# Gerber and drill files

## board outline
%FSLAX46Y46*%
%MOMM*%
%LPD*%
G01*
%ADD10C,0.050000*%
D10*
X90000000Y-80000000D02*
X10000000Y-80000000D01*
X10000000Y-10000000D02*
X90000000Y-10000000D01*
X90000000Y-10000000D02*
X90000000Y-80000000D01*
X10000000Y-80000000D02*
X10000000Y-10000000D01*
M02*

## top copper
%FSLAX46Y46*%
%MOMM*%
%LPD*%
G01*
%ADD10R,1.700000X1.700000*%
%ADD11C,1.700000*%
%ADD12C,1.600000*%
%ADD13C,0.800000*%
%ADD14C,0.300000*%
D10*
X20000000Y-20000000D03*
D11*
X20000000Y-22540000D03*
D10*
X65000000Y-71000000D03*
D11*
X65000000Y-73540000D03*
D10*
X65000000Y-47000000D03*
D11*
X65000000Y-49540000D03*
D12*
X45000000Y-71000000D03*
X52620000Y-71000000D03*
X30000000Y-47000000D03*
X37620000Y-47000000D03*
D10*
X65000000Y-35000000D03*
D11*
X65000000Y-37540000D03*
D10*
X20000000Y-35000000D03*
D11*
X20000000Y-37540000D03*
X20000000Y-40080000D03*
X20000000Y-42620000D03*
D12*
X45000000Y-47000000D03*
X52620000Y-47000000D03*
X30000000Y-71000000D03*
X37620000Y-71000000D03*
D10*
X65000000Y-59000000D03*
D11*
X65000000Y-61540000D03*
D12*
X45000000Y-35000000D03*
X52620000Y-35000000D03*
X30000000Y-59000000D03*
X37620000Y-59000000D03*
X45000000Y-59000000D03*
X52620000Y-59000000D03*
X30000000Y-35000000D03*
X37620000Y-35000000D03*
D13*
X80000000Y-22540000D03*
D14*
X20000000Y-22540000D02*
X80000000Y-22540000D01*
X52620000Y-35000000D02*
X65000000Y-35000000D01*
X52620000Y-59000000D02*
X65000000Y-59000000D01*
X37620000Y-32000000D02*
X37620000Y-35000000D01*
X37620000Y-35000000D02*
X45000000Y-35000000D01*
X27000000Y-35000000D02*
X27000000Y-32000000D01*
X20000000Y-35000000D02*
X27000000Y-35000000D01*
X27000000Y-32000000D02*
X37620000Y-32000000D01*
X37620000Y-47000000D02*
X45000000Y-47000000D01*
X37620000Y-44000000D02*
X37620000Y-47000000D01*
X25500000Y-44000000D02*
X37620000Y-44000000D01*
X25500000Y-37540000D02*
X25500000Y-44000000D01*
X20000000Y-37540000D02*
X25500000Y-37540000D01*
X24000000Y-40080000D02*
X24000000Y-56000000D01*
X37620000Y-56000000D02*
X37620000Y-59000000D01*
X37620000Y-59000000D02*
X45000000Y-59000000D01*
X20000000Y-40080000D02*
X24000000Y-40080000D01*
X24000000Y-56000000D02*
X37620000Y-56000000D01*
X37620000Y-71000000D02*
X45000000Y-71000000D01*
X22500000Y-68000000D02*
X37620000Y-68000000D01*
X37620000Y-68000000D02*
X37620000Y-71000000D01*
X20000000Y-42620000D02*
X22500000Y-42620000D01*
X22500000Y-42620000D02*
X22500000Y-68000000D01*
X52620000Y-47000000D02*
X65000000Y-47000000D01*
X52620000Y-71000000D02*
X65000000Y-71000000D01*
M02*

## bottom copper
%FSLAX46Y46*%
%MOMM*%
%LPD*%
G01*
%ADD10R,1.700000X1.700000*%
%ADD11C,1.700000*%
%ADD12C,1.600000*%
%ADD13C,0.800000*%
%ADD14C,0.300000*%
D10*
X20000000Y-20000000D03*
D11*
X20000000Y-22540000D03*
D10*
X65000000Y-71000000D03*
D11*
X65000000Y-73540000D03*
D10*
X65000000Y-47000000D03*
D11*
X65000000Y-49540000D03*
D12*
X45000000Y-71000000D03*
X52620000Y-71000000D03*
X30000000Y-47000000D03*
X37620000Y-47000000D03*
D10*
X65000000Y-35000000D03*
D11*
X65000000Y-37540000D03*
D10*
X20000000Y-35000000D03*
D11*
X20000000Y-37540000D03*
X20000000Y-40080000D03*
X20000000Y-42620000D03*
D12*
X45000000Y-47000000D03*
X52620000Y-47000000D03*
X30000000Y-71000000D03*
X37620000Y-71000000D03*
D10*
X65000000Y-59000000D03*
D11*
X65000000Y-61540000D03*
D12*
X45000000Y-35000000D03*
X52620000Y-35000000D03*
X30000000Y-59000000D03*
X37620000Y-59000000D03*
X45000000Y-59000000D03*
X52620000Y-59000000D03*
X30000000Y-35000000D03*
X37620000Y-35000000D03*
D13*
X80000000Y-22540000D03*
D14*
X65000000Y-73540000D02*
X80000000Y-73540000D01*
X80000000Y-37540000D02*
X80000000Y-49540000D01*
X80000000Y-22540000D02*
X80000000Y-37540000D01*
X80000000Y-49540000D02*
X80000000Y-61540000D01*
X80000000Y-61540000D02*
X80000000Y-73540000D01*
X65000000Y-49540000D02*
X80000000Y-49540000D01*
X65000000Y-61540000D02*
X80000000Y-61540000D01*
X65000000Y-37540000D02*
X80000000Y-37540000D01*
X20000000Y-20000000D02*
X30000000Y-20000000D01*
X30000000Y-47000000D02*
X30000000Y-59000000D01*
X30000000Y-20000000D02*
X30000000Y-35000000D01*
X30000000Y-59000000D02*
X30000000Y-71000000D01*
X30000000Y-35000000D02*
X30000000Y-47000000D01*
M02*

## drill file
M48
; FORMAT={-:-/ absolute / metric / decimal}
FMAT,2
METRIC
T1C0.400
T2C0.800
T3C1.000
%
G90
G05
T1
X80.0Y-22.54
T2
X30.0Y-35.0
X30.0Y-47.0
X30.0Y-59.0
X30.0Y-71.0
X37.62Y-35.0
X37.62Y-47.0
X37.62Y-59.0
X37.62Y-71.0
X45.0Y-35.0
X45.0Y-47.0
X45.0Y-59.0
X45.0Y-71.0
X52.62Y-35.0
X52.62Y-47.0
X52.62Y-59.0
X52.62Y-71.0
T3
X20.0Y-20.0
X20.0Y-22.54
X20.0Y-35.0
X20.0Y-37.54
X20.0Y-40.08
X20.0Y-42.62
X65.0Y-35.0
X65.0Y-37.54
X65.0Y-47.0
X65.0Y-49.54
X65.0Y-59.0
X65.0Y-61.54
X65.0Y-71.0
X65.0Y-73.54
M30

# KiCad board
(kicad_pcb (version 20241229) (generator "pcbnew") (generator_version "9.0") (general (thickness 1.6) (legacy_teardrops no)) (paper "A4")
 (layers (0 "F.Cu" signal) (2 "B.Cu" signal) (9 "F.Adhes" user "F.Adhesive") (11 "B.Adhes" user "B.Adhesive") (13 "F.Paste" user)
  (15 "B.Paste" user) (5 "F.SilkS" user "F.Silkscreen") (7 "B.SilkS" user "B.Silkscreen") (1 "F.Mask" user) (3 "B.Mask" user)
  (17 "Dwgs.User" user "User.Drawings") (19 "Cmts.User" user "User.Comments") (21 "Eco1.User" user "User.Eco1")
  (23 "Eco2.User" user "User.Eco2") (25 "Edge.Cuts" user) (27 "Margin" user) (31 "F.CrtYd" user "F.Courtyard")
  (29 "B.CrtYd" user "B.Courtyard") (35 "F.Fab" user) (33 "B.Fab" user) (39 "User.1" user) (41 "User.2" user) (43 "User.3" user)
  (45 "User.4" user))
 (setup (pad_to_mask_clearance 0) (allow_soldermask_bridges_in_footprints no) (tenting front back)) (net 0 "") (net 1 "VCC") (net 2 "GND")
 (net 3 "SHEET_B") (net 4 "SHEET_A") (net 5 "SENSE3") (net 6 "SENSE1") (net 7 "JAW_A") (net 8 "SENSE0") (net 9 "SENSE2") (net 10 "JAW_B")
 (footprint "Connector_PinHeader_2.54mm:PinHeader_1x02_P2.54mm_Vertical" (layer "F.Cu") (at 20 20)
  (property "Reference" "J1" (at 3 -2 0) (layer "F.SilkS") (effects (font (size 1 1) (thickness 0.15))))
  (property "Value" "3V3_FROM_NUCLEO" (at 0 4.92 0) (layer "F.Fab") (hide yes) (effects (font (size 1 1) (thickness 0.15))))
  (pad "1" thru_hole rect (at 0 0) (size 1.7 1.7) (drill 1) (layers "*.Cu" "*.Mask") (remove_unused_layers no) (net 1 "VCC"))
  (pad "2" thru_hole circle (at 0 2.54) (size 1.7 1.7) (drill 1) (layers "*.Cu" "*.Mask") (remove_unused_layers no) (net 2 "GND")))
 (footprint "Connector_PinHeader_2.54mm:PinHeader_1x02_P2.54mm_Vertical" (layer "F.Cu") (at 65 71)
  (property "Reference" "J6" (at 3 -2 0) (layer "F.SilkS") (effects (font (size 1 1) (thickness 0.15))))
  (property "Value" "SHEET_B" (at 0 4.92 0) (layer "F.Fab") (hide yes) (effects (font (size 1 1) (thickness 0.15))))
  (pad "1" thru_hole rect (at 0 0) (size 1.7 1.7) (drill 1) (layers "*.Cu" "*.Mask") (remove_unused_layers no) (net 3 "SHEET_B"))
  (pad "2" thru_hole circle (at 0 2.54) (size 1.7 1.7) (drill 1) (layers "*.Cu" "*.Mask") (remove_unused_layers no) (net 2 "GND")))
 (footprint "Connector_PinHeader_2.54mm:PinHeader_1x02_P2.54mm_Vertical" (layer "F.Cu") (at 65 47)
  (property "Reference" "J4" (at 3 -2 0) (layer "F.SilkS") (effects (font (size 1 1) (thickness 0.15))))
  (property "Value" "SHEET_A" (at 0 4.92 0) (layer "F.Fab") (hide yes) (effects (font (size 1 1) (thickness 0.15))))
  (pad "1" thru_hole rect (at 0 0) (size 1.7 1.7) (drill 1) (layers "*.Cu" "*.Mask") (remove_unused_layers no) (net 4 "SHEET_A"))
  (pad "2" thru_hole circle (at 0 2.54) (size 1.7 1.7) (drill 1) (layers "*.Cu" "*.Mask") (remove_unused_layers no) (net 2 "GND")))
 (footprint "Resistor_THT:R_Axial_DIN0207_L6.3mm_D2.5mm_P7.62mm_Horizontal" (layer "F.Cu") (at 45 71)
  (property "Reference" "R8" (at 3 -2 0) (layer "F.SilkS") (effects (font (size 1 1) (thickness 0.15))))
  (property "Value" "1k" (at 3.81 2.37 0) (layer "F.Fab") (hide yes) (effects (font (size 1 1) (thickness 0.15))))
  (pad "1" thru_hole circle (at 0 0) (size 1.6 1.6) (drill 0.8) (layers "*.Cu" "*.Mask") (remove_unused_layers no) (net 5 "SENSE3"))
  (pad "2" thru_hole circle (at 7.62 0) (size 1.6 1.6) (drill 0.8) (layers "*.Cu" "*.Mask") (remove_unused_layers no) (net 3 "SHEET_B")))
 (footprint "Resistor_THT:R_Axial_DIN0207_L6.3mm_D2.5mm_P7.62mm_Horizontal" (layer "F.Cu") (at 30 47)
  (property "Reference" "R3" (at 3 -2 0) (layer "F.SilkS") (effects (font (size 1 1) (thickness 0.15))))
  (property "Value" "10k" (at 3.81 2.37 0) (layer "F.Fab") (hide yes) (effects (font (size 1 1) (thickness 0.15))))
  (pad "1" thru_hole circle (at 0 0) (size 1.6 1.6) (drill 0.8) (layers "*.Cu" "*.Mask") (remove_unused_layers no) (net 1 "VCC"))
  (pad "2" thru_hole circle (at 7.62 0) (size 1.6 1.6) (drill 0.8) (layers "*.Cu" "*.Mask") (remove_unused_layers no) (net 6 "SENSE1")))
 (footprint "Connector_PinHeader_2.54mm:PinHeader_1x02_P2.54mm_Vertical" (layer "F.Cu") (at 65 35)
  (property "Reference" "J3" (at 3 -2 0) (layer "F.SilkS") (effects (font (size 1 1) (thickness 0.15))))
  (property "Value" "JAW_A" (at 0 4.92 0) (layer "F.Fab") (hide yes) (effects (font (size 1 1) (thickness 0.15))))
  (pad "1" thru_hole rect (at 0 0) (size 1.7 1.7) (drill 1) (layers "*.Cu" "*.Mask") (remove_unused_layers no) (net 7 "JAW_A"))
  (pad "2" thru_hole circle (at 0 2.54) (size 1.7 1.7) (drill 1) (layers "*.Cu" "*.Mask") (remove_unused_layers no) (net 2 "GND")))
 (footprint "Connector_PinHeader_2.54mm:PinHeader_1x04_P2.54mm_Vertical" (layer "F.Cu") (at 20 35)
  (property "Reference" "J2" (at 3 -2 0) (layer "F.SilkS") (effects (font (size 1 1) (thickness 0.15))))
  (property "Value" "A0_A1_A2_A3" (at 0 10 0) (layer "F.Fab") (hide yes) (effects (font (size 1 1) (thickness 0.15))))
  (pad "1" thru_hole rect (at 0 0) (size 1.7 1.7) (drill 1) (layers "*.Cu" "*.Mask") (remove_unused_layers no) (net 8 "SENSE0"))
  (pad "2" thru_hole circle (at 0 2.54) (size 1.7 1.7) (drill 1) (layers "*.Cu" "*.Mask") (remove_unused_layers no) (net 6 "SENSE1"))
  (pad "3" thru_hole circle (at 0 5.08) (size 1.7 1.7) (drill 1) (layers "*.Cu" "*.Mask") (remove_unused_layers no) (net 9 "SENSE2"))
  (pad "4" thru_hole circle (at 0 7.62) (size 1.7 1.7) (drill 1) (layers "*.Cu" "*.Mask") (remove_unused_layers no) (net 5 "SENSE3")))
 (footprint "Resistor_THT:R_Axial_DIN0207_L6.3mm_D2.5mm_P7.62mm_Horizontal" (layer "F.Cu") (at 45 47)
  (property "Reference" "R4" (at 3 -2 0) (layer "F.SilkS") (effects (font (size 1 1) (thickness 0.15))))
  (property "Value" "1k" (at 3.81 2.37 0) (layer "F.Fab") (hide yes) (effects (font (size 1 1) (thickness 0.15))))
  (pad "1" thru_hole circle (at 0 0) (size 1.6 1.6) (drill 0.8) (layers "*.Cu" "*.Mask") (remove_unused_layers no) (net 6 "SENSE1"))
  (pad "2" thru_hole circle (at 7.62 0) (size 1.6 1.6) (drill 0.8) (layers "*.Cu" "*.Mask") (remove_unused_layers no) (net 4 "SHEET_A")))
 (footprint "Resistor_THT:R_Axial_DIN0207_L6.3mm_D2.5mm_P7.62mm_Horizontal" (layer "F.Cu") (at 30 71)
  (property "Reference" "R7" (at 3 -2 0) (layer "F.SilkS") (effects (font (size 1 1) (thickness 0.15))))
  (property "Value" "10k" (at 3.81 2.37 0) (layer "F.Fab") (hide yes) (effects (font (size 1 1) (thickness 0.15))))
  (pad "1" thru_hole circle (at 0 0) (size 1.6 1.6) (drill 0.8) (layers "*.Cu" "*.Mask") (remove_unused_layers no) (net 1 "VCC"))
  (pad "2" thru_hole circle (at 7.62 0) (size 1.6 1.6) (drill 0.8) (layers "*.Cu" "*.Mask") (remove_unused_layers no) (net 5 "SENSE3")))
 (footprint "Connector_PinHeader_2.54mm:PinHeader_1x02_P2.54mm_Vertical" (layer "F.Cu") (at 65 59)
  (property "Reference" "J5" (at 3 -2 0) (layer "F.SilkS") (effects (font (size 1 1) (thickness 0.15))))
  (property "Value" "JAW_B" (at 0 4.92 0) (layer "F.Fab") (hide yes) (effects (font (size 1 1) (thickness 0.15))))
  (pad "1" thru_hole rect (at 0 0) (size 1.7 1.7) (drill 1) (layers "*.Cu" "*.Mask") (remove_unused_layers no) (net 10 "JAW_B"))
  (pad "2" thru_hole circle (at 0 2.54) (size 1.7 1.7) (drill 1) (layers "*.Cu" "*.Mask") (remove_unused_layers no) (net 2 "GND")))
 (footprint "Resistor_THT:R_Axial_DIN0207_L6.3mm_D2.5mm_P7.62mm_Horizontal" (layer "F.Cu") (at 45 35)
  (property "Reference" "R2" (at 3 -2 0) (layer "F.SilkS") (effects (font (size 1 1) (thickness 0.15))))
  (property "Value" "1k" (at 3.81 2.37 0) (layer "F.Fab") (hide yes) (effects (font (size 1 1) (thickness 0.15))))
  (pad "1" thru_hole circle (at 0 0) (size 1.6 1.6) (drill 0.8) (layers "*.Cu" "*.Mask") (remove_unused_layers no) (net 8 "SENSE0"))
  (pad "2" thru_hole circle (at 7.62 0) (size 1.6 1.6) (drill 0.8) (layers "*.Cu" "*.Mask") (remove_unused_layers no) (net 7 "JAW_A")))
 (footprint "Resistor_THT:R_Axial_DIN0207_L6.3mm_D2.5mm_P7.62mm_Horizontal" (layer "F.Cu") (at 30 59)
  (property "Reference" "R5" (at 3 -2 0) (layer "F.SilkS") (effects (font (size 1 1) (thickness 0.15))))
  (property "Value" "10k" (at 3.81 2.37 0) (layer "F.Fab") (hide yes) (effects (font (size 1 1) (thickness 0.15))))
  (pad "1" thru_hole circle (at 0 0) (size 1.6 1.6) (drill 0.8) (layers "*.Cu" "*.Mask") (remove_unused_layers no) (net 1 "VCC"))
  (pad "2" thru_hole circle (at 7.62 0) (size 1.6 1.6) (drill 0.8) (layers "*.Cu" "*.Mask") (remove_unused_layers no) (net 9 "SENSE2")))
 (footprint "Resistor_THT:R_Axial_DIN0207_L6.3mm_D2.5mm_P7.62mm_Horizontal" (layer "F.Cu") (at 45 59)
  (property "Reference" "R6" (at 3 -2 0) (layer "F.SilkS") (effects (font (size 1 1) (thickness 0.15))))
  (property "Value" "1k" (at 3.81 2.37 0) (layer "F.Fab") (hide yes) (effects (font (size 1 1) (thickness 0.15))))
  (pad "1" thru_hole circle (at 0 0) (size 1.6 1.6) (drill 0.8) (layers "*.Cu" "*.Mask") (remove_unused_layers no) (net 9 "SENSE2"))
  (pad "2" thru_hole circle (at 7.62 0) (size 1.6 1.6) (drill 0.8) (layers "*.Cu" "*.Mask") (remove_unused_layers no) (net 10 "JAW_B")))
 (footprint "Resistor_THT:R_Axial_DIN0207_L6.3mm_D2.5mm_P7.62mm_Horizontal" (layer "F.Cu") (at 30 35)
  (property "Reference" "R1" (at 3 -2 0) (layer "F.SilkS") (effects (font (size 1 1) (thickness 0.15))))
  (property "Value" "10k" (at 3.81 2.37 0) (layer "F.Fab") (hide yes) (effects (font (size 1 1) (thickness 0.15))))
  (pad "1" thru_hole circle (at 0 0) (size 1.6 1.6) (drill 0.8) (layers "*.Cu" "*.Mask") (remove_unused_layers no) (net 1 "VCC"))
  (pad "2" thru_hole circle (at 7.62 0) (size 1.6 1.6) (drill 0.8) (layers "*.Cu" "*.Mask") (remove_unused_layers no) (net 8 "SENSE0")))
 (gr_line (start 90 80) (end 10 80) (stroke (width 0.05) (type default)) (layer "Edge.Cuts"))
 (gr_line (start 10 10) (end 90 10) (stroke (width 0.05) (type default)) (layer "Edge.Cuts"))
 (gr_line (start 90 10) (end 90 80) (stroke (width 0.05) (type default)) (layer "Edge.Cuts"))
 (gr_line (start 10 80) (end 10 10) (stroke (width 0.05) (type default)) (layer "Edge.Cuts"))
 (segment (start 20 22.54) (end 80 22.54) (width 0.3) (layer "F.Cu") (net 2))
 (via (at 80 22.54) (size 0.8) (drill 0.4) (layers "F.Cu" "B.Cu") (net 2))
 (segment (start 65 73.54) (end 80 73.54) (width 0.3) (layer "B.Cu") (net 2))
 (segment (start 80 37.54) (end 80 49.54) (width 0.3) (layer "B.Cu") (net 2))
 (segment (start 80 22.54) (end 80 37.54) (width 0.3) (layer "B.Cu") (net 2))
 (segment (start 80 49.54) (end 80 61.54) (width 0.3) (layer "B.Cu") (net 2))
 (segment (start 80 61.54) (end 80 73.54) (width 0.3) (layer "B.Cu") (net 2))
 (segment (start 65 49.54) (end 80 49.54) (width 0.3) (layer "B.Cu") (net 2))
 (segment (start 65 61.54) (end 80 61.54) (width 0.3) (layer "B.Cu") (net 2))
 (segment (start 65 37.54) (end 80 37.54) (width 0.3) (layer "B.Cu") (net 2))
 (segment (start 52.62 35) (end 65 35) (width 0.3) (layer "F.Cu") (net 7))
 (segment (start 52.62 59) (end 65 59) (width 0.3) (layer "F.Cu") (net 10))
 (segment (start 37.62 32) (end 37.62 35) (width 0.3) (layer "F.Cu") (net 8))
 (segment (start 37.62 35) (end 45 35) (width 0.3) (layer "F.Cu") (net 8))
 (segment (start 27 35) (end 27 32) (width 0.3) (layer "F.Cu") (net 8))
 (segment (start 20 35) (end 27 35) (width 0.3) (layer "F.Cu") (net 8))
 (segment (start 27 32) (end 37.62 32) (width 0.3) (layer "F.Cu") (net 8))
 (segment (start 37.62 47) (end 45 47) (width 0.3) (layer "F.Cu") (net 6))
 (segment (start 37.62 44) (end 37.62 47) (width 0.3) (layer "F.Cu") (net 6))
 (segment (start 25.5 44) (end 37.62 44) (width 0.3) (layer "F.Cu") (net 6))
 (segment (start 25.5 37.54) (end 25.5 44) (width 0.3) (layer "F.Cu") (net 6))
 (segment (start 20 37.54) (end 25.5 37.54) (width 0.3) (layer "F.Cu") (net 6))
 (segment (start 24 40.08) (end 24 56) (width 0.3) (layer "F.Cu") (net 9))
 (segment (start 37.62 56) (end 37.62 59) (width 0.3) (layer "F.Cu") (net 9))
 (segment (start 37.62 59) (end 45 59) (width 0.3) (layer "F.Cu") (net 9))
 (segment (start 20 40.08) (end 24 40.08) (width 0.3) (layer "F.Cu") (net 9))
 (segment (start 24 56) (end 37.62 56) (width 0.3) (layer "F.Cu") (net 9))
 (segment (start 37.62 71) (end 45 71) (width 0.3) (layer "F.Cu") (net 5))
 (segment (start 22.5 68) (end 37.62 68) (width 0.3) (layer "F.Cu") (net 5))
 (segment (start 37.62 68) (end 37.62 71) (width 0.3) (layer "F.Cu") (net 5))
 (segment (start 20 42.62) (end 22.5 42.62) (width 0.3) (layer "F.Cu") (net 5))
 (segment (start 22.5 42.62) (end 22.5 68) (width 0.3) (layer "F.Cu") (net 5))
 (segment (start 52.62 47) (end 65 47) (width 0.3) (layer "F.Cu") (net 4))
 (segment (start 52.62 71) (end 65 71) (width 0.3) (layer "F.Cu") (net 3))
 (segment (start 20 20) (end 30 20) (width 0.3) (layer "B.Cu") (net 1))
 (segment (start 30 47) (end 30 59) (width 0.3) (layer "B.Cu") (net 1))
 (segment (start 30 20) (end 30 35) (width 0.3) (layer "B.Cu") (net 1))
 (segment (start 30 59) (end 30 71) (width 0.3) (layer "B.Cu") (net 1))
 (segment (start 30 35) (end 30 47) (width 0.3) (layer "B.Cu") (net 1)))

